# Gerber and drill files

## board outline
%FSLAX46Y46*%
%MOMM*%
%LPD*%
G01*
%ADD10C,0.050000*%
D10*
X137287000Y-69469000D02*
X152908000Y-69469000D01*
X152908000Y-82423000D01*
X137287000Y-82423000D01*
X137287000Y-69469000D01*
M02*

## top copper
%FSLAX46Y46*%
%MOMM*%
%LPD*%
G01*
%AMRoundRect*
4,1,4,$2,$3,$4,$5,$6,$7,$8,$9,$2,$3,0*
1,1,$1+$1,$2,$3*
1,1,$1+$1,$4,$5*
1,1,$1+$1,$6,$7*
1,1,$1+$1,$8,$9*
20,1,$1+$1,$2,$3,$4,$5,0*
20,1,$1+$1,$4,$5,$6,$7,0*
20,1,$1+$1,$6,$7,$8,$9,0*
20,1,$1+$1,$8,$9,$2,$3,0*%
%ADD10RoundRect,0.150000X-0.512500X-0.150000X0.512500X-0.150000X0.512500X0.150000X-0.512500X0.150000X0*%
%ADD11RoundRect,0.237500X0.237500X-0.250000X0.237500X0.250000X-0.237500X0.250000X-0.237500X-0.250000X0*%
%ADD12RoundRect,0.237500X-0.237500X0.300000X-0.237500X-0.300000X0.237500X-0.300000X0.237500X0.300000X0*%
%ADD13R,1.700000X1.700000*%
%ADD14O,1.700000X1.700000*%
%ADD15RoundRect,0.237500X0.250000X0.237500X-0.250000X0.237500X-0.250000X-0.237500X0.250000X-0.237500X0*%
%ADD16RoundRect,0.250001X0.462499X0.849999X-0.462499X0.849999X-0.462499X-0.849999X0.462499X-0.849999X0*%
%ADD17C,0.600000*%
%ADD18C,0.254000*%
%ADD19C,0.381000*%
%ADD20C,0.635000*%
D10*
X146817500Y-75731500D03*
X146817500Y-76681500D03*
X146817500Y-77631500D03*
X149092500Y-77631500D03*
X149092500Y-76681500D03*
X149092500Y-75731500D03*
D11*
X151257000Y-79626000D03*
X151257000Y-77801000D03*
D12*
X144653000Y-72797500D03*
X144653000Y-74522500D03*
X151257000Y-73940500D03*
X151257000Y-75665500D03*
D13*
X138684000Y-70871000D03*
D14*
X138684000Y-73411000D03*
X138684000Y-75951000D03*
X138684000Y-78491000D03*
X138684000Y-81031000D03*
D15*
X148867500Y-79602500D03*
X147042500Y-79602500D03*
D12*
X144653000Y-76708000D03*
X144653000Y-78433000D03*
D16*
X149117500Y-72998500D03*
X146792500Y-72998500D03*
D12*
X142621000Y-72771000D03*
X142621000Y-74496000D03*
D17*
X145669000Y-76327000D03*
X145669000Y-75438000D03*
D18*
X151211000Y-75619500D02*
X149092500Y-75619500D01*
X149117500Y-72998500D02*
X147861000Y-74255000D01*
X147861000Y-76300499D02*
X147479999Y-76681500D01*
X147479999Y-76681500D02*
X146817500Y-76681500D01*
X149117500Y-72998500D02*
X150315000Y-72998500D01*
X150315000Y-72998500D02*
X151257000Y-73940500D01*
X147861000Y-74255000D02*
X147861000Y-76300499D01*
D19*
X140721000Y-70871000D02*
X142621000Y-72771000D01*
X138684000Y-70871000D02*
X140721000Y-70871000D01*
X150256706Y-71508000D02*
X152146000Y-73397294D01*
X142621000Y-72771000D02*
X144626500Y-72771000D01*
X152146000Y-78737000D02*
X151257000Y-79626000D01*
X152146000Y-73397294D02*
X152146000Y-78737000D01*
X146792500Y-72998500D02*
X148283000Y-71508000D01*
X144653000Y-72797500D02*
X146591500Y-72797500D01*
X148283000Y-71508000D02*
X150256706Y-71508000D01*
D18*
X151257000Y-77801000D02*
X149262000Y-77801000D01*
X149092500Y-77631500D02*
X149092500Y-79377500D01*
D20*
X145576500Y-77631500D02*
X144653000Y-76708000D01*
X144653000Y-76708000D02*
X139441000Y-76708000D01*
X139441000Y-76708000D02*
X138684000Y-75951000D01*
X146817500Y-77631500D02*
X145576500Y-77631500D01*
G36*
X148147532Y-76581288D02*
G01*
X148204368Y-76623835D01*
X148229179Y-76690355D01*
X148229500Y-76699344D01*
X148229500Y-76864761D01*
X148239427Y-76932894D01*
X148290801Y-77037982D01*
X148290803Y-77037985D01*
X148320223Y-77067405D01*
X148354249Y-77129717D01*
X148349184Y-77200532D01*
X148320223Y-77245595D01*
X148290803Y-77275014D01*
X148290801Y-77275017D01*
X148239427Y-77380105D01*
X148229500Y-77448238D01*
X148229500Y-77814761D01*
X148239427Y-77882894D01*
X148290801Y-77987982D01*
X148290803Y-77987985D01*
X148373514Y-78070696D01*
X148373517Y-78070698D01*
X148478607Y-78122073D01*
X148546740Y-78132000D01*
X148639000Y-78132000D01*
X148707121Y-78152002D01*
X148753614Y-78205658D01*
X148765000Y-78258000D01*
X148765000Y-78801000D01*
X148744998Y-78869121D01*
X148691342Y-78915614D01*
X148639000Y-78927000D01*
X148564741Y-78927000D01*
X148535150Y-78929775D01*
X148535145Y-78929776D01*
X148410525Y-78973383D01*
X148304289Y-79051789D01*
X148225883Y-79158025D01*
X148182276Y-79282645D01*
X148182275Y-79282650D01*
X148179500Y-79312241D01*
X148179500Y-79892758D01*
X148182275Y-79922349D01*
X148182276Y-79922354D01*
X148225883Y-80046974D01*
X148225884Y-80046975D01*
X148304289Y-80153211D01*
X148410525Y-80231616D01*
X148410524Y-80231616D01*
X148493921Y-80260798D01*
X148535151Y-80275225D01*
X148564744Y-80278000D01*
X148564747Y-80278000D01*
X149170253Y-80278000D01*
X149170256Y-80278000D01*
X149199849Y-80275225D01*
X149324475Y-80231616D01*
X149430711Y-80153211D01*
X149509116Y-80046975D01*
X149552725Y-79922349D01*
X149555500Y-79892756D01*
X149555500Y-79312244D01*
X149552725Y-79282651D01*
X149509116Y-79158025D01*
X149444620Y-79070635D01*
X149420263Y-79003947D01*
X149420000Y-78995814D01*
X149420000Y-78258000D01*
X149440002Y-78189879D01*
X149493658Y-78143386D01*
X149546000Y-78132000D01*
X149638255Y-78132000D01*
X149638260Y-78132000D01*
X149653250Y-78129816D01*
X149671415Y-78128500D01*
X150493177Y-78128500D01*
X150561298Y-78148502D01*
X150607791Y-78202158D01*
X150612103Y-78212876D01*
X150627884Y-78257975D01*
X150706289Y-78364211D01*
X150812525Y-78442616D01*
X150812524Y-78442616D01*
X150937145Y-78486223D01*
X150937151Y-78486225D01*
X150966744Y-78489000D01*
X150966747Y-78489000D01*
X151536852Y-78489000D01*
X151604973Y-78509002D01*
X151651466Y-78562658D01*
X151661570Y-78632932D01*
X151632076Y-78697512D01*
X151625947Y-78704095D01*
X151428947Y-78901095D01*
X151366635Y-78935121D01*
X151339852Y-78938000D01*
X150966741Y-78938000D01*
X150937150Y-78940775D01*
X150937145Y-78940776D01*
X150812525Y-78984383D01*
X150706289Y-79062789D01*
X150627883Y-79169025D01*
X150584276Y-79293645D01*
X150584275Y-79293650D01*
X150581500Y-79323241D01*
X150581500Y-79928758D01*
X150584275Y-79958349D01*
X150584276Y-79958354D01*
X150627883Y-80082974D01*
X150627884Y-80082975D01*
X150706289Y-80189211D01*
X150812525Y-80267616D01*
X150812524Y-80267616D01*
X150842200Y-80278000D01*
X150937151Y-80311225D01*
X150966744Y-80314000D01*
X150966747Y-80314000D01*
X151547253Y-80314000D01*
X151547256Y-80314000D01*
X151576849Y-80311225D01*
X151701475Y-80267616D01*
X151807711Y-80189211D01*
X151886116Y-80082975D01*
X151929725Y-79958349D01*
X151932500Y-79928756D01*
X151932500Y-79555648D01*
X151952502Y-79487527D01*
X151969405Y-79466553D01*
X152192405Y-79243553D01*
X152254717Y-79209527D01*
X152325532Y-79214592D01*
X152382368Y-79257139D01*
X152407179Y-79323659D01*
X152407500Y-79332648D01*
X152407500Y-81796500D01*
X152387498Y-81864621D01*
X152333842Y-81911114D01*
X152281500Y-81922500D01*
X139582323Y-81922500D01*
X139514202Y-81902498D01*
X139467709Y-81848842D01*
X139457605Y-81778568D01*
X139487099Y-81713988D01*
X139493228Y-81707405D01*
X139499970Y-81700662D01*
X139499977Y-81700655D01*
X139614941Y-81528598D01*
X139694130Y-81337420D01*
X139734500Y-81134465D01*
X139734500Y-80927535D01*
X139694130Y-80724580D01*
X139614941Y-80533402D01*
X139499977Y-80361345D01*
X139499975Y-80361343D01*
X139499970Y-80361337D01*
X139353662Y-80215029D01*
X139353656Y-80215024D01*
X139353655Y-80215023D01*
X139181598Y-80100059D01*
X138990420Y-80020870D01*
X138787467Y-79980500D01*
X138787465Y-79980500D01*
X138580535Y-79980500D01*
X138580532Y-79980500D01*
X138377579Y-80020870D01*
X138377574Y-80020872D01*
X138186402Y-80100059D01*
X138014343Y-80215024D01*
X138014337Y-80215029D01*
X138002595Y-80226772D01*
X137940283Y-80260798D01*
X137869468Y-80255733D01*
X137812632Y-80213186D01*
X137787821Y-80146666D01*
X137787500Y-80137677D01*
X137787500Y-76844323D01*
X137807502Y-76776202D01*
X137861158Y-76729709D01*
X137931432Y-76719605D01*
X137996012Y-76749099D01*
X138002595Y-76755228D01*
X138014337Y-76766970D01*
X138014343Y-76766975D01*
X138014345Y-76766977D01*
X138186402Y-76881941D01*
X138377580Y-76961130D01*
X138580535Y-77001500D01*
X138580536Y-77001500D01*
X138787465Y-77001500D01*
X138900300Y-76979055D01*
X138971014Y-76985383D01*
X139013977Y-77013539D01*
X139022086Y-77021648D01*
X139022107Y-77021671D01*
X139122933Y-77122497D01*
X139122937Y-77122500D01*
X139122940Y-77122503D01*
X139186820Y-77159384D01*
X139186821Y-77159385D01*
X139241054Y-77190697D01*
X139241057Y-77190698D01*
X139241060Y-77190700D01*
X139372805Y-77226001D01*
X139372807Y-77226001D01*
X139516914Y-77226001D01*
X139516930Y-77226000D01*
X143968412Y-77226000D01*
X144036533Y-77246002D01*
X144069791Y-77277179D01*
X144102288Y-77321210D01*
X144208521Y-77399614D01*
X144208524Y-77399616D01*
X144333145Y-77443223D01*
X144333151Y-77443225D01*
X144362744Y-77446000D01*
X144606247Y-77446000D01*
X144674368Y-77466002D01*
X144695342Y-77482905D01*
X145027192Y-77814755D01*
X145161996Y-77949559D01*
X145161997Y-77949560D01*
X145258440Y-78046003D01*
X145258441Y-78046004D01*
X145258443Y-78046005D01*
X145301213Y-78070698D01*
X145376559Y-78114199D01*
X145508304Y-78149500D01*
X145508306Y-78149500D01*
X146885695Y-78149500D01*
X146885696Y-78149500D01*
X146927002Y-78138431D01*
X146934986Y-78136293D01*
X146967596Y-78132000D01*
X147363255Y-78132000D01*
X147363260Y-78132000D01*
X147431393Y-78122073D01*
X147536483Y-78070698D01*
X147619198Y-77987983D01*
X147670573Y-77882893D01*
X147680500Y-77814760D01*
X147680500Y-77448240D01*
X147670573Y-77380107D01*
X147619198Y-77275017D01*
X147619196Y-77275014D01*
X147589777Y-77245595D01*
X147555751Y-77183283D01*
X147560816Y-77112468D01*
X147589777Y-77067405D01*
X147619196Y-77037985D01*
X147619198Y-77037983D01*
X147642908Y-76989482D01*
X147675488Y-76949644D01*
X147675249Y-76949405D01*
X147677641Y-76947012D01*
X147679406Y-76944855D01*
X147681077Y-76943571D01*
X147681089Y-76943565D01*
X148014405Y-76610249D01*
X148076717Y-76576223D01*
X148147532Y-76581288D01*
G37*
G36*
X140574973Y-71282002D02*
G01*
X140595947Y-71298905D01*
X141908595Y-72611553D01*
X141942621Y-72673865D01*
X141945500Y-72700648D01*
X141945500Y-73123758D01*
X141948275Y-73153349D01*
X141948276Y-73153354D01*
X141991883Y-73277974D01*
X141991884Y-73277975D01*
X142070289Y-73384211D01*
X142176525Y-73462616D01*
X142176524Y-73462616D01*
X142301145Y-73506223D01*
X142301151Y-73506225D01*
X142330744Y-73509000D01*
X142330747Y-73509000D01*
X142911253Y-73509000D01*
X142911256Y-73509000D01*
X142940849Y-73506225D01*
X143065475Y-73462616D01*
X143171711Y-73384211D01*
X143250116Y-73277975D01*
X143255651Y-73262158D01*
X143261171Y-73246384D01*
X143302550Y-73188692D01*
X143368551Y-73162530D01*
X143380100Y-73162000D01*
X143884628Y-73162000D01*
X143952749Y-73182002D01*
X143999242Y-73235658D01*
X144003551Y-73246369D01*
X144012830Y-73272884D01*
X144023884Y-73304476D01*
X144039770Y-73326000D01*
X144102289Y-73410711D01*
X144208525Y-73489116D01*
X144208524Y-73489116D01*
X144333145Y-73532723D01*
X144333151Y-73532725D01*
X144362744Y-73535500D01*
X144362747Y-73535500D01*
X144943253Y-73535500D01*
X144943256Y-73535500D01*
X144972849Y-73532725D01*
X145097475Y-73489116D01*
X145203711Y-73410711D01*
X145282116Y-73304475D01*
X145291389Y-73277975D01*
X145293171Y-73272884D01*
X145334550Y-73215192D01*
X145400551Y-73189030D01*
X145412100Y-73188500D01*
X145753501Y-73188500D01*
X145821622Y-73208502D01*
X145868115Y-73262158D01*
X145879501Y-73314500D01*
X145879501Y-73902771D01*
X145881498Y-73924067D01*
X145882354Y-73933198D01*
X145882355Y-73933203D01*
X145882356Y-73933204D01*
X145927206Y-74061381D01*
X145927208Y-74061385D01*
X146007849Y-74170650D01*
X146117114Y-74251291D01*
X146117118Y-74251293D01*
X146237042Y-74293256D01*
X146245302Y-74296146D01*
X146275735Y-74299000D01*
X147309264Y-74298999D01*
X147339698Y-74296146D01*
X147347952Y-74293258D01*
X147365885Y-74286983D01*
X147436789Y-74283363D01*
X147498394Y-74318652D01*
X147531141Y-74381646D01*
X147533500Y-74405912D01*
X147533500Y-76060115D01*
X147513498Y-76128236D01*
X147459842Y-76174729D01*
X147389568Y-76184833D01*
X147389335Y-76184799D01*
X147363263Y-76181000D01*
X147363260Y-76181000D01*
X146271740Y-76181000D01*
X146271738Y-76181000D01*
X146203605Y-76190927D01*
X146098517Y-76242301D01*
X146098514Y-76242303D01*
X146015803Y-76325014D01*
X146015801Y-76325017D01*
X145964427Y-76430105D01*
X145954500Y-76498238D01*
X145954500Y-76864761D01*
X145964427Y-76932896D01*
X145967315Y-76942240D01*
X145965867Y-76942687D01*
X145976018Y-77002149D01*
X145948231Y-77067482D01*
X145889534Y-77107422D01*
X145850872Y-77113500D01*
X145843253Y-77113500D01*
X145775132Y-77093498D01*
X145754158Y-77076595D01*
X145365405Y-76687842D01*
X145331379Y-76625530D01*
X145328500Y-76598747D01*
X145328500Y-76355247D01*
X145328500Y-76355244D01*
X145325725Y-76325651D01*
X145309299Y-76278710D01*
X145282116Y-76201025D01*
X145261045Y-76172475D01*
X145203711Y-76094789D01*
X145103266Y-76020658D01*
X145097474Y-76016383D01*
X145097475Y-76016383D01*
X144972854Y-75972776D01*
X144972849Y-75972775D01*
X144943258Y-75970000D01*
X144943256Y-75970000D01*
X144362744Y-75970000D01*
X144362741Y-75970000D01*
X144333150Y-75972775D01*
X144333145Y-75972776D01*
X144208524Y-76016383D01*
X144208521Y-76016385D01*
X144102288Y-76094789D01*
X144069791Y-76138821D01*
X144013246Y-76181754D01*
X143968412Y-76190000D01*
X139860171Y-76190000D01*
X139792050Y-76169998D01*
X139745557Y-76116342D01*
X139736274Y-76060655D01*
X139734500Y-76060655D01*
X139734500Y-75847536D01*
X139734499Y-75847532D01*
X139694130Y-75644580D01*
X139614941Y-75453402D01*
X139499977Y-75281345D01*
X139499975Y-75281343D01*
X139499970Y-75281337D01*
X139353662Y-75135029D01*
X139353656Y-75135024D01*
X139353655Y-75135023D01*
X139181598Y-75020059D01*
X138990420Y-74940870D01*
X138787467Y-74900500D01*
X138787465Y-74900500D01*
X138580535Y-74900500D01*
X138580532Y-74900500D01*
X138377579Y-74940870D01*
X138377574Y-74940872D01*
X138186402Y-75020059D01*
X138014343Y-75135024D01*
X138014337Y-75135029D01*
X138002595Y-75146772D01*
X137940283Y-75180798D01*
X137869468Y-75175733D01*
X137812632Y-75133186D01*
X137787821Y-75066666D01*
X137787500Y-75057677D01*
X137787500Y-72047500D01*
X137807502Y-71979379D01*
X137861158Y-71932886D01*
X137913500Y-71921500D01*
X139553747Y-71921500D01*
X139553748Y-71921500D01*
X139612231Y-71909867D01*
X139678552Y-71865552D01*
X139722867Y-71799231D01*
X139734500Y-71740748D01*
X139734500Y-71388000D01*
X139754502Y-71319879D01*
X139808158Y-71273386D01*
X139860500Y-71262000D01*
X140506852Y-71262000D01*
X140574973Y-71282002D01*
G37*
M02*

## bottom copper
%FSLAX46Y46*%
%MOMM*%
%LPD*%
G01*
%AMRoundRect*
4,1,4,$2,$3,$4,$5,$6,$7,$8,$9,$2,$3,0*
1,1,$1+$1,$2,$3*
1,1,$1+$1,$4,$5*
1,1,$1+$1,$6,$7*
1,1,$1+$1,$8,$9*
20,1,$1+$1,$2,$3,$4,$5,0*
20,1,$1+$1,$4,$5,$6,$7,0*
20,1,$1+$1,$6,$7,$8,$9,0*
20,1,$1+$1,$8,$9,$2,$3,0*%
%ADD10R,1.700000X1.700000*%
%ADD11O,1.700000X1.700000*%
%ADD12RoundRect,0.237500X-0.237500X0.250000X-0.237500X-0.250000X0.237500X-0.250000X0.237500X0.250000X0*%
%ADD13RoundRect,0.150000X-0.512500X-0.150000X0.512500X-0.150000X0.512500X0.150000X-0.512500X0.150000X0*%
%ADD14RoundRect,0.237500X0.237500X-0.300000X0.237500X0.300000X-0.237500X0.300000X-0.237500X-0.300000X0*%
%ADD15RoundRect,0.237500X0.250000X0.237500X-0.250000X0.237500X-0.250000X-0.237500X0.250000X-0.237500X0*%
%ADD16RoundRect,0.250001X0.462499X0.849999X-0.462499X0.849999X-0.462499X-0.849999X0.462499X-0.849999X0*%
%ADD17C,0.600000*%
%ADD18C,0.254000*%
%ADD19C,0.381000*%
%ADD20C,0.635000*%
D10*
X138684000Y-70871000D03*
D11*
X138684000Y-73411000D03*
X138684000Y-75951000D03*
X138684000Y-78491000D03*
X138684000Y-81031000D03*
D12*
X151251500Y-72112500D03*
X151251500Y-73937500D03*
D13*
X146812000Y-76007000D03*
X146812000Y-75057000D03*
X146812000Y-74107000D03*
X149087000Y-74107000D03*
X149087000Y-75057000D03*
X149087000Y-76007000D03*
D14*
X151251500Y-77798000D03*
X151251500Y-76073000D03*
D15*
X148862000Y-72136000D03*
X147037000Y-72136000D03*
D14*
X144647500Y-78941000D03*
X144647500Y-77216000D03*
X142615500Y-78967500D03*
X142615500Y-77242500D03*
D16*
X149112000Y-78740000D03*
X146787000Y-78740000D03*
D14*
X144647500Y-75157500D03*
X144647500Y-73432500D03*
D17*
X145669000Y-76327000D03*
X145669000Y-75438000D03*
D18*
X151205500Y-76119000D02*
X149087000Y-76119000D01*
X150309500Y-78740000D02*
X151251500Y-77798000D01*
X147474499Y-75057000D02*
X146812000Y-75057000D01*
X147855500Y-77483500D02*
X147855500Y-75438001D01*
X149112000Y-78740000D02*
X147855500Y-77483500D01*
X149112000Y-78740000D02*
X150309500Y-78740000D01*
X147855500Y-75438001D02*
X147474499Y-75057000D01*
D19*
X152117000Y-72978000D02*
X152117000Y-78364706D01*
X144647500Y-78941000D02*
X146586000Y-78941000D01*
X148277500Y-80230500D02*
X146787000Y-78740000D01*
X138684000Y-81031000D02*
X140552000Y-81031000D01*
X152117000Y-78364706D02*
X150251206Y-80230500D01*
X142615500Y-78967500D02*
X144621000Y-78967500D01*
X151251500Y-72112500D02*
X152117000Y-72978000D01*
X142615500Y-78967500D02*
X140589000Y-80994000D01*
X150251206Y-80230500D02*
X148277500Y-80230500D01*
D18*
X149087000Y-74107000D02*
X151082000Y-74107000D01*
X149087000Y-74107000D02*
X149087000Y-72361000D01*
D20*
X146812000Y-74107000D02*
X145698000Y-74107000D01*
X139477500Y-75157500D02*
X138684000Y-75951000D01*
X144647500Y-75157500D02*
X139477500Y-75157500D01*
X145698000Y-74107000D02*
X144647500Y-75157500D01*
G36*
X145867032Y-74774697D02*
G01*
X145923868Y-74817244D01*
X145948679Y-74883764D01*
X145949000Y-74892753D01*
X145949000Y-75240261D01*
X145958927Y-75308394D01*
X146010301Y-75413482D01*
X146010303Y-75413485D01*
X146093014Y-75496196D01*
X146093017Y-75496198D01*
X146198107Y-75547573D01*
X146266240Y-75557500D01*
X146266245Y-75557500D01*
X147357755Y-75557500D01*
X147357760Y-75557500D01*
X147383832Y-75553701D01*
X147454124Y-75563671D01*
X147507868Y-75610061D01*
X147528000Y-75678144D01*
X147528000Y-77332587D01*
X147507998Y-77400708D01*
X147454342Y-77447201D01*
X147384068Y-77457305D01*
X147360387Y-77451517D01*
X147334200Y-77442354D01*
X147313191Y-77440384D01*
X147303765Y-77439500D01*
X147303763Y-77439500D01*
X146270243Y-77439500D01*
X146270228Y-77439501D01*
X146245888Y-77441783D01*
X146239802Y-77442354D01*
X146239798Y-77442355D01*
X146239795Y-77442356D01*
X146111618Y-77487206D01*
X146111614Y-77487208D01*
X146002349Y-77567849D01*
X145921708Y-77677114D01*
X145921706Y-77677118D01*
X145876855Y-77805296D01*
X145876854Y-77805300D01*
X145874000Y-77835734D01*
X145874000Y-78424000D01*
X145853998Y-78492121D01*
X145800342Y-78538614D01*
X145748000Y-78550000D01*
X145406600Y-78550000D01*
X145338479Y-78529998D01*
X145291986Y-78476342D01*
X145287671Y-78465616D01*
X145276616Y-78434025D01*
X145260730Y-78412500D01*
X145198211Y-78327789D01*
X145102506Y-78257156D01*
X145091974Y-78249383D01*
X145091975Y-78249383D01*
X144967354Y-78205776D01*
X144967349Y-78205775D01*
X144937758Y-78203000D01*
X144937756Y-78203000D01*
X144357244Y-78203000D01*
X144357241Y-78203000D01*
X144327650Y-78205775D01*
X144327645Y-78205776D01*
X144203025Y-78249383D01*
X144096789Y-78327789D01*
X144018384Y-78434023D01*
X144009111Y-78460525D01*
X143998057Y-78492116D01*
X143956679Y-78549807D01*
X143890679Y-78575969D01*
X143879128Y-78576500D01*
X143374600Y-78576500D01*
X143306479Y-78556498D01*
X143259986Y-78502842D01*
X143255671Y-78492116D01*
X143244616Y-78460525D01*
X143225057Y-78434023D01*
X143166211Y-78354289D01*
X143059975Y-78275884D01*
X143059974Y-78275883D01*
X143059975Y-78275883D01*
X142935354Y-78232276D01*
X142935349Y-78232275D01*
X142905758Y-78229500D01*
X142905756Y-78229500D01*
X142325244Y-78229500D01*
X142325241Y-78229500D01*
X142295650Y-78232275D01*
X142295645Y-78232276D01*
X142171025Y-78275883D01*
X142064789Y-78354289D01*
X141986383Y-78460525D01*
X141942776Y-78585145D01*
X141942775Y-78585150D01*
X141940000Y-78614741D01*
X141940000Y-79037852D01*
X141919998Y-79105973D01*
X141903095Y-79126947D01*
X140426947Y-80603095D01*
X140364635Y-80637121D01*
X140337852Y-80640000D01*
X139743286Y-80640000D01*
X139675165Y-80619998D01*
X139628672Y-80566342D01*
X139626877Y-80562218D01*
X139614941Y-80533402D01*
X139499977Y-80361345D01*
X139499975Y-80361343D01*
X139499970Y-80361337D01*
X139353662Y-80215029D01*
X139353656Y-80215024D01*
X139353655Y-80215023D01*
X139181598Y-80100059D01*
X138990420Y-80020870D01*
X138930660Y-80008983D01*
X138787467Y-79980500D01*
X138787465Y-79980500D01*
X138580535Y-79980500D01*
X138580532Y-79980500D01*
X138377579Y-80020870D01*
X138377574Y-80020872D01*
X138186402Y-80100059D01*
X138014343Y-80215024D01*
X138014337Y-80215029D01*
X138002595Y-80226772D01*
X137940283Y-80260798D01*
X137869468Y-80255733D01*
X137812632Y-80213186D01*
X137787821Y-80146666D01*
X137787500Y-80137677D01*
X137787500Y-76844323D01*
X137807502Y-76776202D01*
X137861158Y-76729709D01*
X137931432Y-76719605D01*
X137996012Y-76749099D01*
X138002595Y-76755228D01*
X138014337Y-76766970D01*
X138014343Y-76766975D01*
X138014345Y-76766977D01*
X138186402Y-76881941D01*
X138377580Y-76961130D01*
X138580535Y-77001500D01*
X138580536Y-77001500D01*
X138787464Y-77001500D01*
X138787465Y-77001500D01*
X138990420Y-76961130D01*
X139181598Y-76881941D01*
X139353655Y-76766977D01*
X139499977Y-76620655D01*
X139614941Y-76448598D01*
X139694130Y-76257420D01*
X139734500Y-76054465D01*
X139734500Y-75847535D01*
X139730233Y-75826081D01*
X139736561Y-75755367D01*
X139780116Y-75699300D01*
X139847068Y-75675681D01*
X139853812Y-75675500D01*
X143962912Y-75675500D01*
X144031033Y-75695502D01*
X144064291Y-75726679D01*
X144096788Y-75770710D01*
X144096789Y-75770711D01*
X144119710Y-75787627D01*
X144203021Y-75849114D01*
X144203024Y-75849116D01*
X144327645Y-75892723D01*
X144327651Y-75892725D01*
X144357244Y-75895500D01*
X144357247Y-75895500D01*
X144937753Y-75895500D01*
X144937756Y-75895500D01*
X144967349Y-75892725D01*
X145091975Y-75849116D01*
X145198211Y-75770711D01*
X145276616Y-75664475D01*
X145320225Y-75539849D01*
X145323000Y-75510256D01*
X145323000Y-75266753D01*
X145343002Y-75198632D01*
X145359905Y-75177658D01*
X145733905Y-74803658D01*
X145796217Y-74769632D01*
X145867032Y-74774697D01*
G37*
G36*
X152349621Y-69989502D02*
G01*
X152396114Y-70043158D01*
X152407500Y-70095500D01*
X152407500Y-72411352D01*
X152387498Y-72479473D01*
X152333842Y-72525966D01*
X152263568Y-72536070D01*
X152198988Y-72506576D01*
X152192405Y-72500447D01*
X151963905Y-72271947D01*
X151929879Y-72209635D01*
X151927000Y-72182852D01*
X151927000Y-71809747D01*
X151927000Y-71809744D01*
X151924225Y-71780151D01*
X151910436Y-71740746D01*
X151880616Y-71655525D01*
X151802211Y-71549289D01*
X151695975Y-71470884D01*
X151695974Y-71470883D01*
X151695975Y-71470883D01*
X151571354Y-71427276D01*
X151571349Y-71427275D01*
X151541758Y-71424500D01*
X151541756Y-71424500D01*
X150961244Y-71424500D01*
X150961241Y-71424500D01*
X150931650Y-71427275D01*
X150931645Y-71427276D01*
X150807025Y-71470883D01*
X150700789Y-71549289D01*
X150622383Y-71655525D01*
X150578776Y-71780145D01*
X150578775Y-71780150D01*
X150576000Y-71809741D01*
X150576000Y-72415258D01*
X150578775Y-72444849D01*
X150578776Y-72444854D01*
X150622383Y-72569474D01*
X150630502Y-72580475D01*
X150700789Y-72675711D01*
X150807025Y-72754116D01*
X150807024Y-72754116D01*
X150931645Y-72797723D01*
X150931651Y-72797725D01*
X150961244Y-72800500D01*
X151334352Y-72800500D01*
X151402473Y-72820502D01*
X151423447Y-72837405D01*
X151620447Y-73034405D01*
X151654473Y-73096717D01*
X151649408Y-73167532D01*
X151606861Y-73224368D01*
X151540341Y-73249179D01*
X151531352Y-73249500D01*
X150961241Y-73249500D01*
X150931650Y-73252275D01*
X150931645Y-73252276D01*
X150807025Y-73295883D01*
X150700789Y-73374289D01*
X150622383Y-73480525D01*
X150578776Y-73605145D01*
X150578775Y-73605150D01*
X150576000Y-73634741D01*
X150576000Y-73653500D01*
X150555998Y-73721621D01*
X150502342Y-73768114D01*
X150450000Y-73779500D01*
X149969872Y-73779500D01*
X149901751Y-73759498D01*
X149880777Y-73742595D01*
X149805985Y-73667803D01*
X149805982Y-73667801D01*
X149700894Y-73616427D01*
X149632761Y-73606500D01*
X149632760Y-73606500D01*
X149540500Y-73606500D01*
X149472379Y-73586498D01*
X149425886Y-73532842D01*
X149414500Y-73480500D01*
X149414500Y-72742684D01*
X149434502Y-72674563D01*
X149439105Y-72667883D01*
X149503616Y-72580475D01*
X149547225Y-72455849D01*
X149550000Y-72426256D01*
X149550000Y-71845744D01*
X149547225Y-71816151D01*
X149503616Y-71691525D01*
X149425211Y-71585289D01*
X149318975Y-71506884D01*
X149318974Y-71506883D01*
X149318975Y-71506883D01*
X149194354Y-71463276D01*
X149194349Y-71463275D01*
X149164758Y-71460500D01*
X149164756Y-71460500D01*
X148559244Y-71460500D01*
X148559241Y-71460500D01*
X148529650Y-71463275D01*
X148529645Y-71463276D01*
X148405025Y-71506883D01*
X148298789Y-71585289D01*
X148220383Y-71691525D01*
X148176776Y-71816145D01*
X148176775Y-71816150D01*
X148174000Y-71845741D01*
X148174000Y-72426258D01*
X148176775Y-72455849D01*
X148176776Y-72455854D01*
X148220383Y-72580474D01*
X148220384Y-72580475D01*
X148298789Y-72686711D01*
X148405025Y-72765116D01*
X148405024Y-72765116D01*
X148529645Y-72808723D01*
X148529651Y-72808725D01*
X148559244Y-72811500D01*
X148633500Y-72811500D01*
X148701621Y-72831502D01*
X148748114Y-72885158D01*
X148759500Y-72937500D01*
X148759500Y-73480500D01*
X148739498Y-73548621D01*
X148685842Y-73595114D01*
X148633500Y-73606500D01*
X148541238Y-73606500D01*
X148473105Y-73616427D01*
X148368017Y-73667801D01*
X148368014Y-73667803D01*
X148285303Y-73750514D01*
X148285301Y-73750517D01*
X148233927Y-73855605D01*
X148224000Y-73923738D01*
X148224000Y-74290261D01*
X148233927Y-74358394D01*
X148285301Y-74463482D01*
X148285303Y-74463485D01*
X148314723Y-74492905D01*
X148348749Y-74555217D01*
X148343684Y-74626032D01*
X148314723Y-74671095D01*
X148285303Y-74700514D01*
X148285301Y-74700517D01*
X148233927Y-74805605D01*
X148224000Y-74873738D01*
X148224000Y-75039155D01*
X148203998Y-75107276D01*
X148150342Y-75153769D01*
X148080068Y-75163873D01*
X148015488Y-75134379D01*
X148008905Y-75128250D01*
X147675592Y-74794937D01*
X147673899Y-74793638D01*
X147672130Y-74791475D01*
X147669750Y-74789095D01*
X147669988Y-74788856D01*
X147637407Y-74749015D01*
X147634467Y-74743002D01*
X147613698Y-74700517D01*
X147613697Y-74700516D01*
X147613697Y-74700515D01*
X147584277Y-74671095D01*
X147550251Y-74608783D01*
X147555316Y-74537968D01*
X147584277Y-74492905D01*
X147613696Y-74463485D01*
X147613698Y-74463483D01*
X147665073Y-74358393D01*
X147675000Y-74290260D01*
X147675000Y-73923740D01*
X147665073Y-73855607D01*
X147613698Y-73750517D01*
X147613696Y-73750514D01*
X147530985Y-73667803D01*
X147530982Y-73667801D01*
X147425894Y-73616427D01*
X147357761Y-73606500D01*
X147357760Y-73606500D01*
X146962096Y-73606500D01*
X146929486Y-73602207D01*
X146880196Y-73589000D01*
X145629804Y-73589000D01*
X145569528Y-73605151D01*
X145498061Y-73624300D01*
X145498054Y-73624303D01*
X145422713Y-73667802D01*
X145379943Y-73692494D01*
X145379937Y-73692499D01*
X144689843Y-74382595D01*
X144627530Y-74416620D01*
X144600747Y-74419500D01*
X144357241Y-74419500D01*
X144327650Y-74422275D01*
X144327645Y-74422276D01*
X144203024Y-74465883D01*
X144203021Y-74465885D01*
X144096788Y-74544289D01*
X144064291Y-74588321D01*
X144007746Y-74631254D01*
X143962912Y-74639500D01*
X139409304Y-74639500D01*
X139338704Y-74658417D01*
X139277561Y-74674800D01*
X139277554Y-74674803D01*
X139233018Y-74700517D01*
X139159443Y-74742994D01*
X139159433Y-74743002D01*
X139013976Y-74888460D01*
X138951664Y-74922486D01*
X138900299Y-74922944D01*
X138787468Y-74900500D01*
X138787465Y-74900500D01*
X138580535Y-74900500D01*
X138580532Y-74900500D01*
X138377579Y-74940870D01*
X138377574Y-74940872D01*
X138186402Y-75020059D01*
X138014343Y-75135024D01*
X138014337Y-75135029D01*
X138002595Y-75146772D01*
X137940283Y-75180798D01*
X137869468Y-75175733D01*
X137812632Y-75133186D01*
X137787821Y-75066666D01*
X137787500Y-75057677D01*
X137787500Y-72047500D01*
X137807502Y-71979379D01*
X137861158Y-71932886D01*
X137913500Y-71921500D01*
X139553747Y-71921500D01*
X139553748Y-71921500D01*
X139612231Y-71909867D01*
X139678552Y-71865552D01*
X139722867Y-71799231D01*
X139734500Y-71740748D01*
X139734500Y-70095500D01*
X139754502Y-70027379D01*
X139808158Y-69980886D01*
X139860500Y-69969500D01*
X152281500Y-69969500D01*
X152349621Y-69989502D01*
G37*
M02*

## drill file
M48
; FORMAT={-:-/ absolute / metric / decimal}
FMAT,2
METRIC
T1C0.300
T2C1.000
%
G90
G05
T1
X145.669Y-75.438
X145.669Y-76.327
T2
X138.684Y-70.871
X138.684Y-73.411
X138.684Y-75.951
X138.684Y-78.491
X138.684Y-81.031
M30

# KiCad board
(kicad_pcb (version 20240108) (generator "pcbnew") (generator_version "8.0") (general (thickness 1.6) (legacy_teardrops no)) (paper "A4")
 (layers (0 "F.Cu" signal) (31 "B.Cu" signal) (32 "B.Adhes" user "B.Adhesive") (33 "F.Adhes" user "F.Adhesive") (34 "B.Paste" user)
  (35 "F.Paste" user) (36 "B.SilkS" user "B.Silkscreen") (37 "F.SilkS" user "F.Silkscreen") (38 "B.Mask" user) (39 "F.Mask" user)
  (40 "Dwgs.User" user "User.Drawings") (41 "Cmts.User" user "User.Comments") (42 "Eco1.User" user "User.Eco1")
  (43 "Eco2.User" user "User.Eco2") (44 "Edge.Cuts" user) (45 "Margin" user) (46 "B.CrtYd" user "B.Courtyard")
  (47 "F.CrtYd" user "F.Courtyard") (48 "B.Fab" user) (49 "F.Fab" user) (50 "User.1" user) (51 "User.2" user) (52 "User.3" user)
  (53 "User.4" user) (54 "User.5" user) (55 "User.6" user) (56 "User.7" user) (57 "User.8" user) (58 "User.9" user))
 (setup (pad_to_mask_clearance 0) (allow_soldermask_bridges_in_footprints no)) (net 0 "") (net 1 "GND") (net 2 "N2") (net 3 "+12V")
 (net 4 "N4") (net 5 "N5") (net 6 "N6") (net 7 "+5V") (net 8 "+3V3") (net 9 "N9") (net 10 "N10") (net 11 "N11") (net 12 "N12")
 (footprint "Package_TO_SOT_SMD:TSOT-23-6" (layer "F.Cu") (at 147.955 76.6815)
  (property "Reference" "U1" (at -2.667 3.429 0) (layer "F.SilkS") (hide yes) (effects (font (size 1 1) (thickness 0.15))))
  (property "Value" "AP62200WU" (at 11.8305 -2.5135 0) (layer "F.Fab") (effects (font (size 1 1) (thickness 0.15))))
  (pad "1" smd roundrect (at -1.1375 -0.95) (size 1.325 0.6) (layers "F.Cu" "F.Paste" "F.Mask") (roundrect_rratio 0.25) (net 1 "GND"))
  (pad "2" smd roundrect (at -1.1375 0) (size 1.325 0.6) (layers "F.Cu" "F.Paste" "F.Mask") (roundrect_rratio 0.25) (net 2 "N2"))
  (pad "3" smd roundrect (at -1.1375 0.95) (size 1.325 0.6) (layers "F.Cu" "F.Paste" "F.Mask") (roundrect_rratio 0.25) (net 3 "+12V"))
  (pad "4" smd roundrect (at 1.1375 0.95) (size 1.325 0.6) (layers "F.Cu" "F.Paste" "F.Mask") (roundrect_rratio 0.25) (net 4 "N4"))
  (pad "5" smd roundrect (at 1.1375 0) (size 1.325 0.6) (layers "F.Cu" "F.Paste" "F.Mask") (roundrect_rratio 0.25) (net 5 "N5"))
  (pad "6" smd roundrect (at 1.1375 -0.95) (size 1.325 0.6) (layers "F.Cu" "F.Paste" "F.Mask") (roundrect_rratio 0.25) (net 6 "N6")))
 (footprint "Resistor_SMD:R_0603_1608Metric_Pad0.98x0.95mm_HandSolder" (layer "F.Cu") (at 151.257 78.7135 90)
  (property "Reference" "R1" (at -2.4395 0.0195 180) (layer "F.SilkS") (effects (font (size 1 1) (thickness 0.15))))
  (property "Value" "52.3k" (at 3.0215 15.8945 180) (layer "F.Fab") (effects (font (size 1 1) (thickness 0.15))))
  (pad "1" smd roundrect (at -0.9125 0 90) (size 0.975 0.95) (layers "F.Cu" "F.Paste" "F.Mask") (roundrect_rratio 0.25) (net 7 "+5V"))
  (pad "2" smd roundrect (at 0.9125 0 90) (size 0.975 0.95) (layers "F.Cu" "F.Paste" "F.Mask") (roundrect_rratio 0.25) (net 4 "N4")))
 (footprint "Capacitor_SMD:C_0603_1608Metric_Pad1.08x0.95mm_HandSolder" (layer "F.Cu") (at 144.653 73.66 -90)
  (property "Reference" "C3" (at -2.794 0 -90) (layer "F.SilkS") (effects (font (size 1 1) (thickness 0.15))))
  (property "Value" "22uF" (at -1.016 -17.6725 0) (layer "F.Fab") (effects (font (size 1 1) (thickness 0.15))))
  (pad "1" smd roundrect (at -0.8625 0 270) (size 1.075 0.95) (layers "F.Cu" "F.Paste" "F.Mask") (roundrect_rratio 0.25) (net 7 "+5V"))
  (pad "2" smd roundrect (at 0.8625 0 270) (size 1.075 0.95) (layers "F.Cu" "F.Paste" "F.Mask") (roundrect_rratio 0.25) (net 1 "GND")))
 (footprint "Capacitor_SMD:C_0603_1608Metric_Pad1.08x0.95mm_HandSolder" (layer "F.Cu") (at 151.257 74.803 -90)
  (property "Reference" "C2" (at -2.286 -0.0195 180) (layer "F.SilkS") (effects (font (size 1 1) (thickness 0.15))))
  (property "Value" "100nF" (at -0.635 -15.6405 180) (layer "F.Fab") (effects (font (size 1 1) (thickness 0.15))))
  (pad "1" smd roundrect (at -0.8625 0 270) (size 1.075 0.95) (layers "F.Cu" "F.Paste" "F.Mask") (roundrect_rratio 0.25) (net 2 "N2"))
  (pad "2" smd roundrect (at 0.8625 0 270) (size 1.075 0.95) (layers "F.Cu" "F.Paste" "F.Mask") (roundrect_rratio 0.25) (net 6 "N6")))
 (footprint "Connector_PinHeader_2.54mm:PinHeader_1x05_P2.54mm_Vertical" (layer "F.Cu") (at 138.684 70.871)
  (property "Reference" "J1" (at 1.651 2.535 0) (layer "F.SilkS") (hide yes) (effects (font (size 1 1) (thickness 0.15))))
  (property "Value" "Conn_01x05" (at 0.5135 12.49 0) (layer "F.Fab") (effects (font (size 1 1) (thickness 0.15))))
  (pad "1" thru_hole rect (at 0 0) (size 1.7 1.7) (drill 1) (layers "*.Cu" "*.Mask") (remove_unused_layers no) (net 7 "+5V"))
  (pad "2" thru_hole oval (at 0 2.54) (size 1.7 1.7) (drill 1) (layers "*.Cu" "*.Mask") (remove_unused_layers no) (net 1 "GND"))
  (pad "3" thru_hole oval (at 0 5.08) (size 1.7 1.7) (drill 1) (layers "*.Cu" "*.Mask") (remove_unused_layers no) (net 3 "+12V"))
  (pad "4" thru_hole oval (at 0 7.62) (size 1.7 1.7) (drill 1) (layers "*.Cu" "*.Mask") (remove_unused_layers no) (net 1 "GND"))
  (pad "5" thru_hole oval (at 0 10.16) (size 1.7 1.7) (drill 1) (layers "*.Cu" "*.Mask") (remove_unused_layers no) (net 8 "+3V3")))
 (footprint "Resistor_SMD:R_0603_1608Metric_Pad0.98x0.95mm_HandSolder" (layer "F.Cu") (at 147.955 79.6025 180)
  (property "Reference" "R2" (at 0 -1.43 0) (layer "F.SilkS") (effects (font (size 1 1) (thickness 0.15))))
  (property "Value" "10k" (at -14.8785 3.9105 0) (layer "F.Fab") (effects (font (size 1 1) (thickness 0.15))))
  (pad "1" smd roundrect (at -0.9125 0 180) (size 0.975 0.95) (layers "F.Cu" "F.Paste" "F.Mask") (roundrect_rratio 0.25) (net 4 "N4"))
  (pad "2" smd roundrect (at 0.9125 0 180) (size 0.975 0.95) (layers "F.Cu" "F.Paste" "F.Mask") (roundrect_rratio 0.25) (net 1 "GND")))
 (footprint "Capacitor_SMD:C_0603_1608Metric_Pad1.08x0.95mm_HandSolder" (layer "F.Cu") (at 144.653 77.5705 -90)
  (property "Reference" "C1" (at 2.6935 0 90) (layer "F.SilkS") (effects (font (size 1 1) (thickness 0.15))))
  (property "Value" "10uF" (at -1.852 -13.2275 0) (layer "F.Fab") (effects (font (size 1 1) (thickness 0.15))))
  (pad "1" smd roundrect (at -0.8625 0 270) (size 1.075 0.95) (layers "F.Cu" "F.Paste" "F.Mask") (roundrect_rratio 0.25) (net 3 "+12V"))
  (pad "2" smd roundrect (at 0.8625 0 270) (size 1.075 0.95) (layers "F.Cu" "F.Paste" "F.Mask") (roundrect_rratio 0.25) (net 1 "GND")))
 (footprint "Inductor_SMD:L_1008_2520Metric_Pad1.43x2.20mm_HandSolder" (layer "F.Cu") (at 147.955 72.9985 180)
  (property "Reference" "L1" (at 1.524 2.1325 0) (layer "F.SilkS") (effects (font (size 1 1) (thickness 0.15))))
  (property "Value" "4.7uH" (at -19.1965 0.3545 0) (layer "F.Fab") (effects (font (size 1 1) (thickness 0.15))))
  (pad "1" smd roundrect (at -1.1625 0 180) (size 1.425 2.2) (layers "F.Cu" "F.Paste" "F.Mask") (roundrect_rratio 0.175439) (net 2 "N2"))
  (pad "2" smd roundrect (at 1.1625 0 180) (size 1.425 2.2) (layers "F.Cu" "F.Paste" "F.Mask") (roundrect_rratio 0.175439) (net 7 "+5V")))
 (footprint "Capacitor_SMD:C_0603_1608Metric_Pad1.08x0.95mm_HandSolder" (layer "F.Cu") (at 142.621 73.6335 -90)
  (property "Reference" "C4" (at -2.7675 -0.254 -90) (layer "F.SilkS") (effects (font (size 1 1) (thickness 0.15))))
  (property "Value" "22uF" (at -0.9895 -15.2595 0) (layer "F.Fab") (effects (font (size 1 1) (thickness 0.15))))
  (pad "1" smd roundrect (at -0.8625 0 270) (size 1.075 0.95) (layers "F.Cu" "F.Paste" "F.Mask") (roundrect_rratio 0.25) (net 7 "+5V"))
  (pad "2" smd roundrect (at 0.8625 0 270) (size 1.075 0.95) (layers "F.Cu" "F.Paste" "F.Mask") (roundrect_rratio 0.25) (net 1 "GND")))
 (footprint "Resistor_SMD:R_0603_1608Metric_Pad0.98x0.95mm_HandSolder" (layer "B.Cu") (at 151.2515 73.025 -90)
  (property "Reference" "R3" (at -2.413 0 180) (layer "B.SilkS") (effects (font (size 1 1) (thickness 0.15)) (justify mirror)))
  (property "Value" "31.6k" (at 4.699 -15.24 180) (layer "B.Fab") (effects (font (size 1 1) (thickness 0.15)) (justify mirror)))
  (pad "1" smd roundrect (at -0.9125 0 270) (size 0.975 0.95) (layers "B.Cu" "B.Paste" "B.Mask") (roundrect_rratio 0.25) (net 8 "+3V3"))
  (pad "2" smd roundrect (at 0.9125 0 270) (size 0.975 0.95) (layers "B.Cu" "B.Paste" "B.Mask") (roundrect_rratio 0.25) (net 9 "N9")))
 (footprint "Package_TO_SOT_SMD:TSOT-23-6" (layer "B.Cu") (at 147.9495 75.057)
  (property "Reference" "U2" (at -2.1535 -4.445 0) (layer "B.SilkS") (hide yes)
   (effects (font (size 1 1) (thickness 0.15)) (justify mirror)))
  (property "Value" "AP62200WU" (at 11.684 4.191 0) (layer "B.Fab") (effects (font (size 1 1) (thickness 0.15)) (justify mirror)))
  (pad "1" smd roundrect (at -1.1375 0.95) (size 1.325 0.6) (layers "B.Cu" "B.Paste" "B.Mask") (roundrect_rratio 0.25) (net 1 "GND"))
  (pad "2" smd roundrect (at -1.1375 0) (size 1.325 0.6) (layers "B.Cu" "B.Paste" "B.Mask") (roundrect_rratio 0.25) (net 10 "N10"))
  (pad "3" smd roundrect (at -1.1375 -0.95) (size 1.325 0.6) (layers "B.Cu" "B.Paste" "B.Mask") (roundrect_rratio 0.25) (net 3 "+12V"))
  (pad "4" smd roundrect (at 1.1375 -0.95) (size 1.325 0.6) (layers "B.Cu" "B.Paste" "B.Mask") (roundrect_rratio 0.25) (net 9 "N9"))
  (pad "5" smd roundrect (at 1.1375 0) (size 1.325 0.6) (layers "B.Cu" "B.Paste" "B.Mask") (roundrect_rratio 0.25) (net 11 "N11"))
  (pad "6" smd roundrect (at 1.1375 0.95) (size 1.325 0.6) (layers "B.Cu" "B.Paste" "B.Mask") (roundrect_rratio 0.25) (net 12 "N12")))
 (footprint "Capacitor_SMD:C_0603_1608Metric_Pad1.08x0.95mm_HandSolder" (layer "B.Cu") (at 151.2515 76.9355 90)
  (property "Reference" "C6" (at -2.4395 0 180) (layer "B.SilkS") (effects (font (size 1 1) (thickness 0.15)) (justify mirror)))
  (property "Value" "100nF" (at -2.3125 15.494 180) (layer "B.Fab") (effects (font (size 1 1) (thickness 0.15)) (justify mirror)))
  (pad "1" smd roundrect (at -0.8625 0 90) (size 1.075 0.95) (layers "B.Cu" "B.Paste" "B.Mask") (roundrect_rratio 0.25) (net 10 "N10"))
  (pad "2" smd roundrect (at 0.8625 0 90) (size 1.075 0.95) (layers "B.Cu" "B.Paste" "B.Mask") (roundrect_rratio 0.25) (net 12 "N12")))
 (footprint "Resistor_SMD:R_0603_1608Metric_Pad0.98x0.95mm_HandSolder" (layer "B.Cu") (at 147.9495 72.136 180)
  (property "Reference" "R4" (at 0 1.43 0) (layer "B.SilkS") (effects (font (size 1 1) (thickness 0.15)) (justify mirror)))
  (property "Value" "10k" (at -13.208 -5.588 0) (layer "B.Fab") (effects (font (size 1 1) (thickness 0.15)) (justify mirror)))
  (pad "1" smd roundrect (at -0.9125 0 180) (size 0.975 0.95) (layers "B.Cu" "B.Paste" "B.Mask") (roundrect_rratio 0.25) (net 9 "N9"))
  (pad "2" smd roundrect (at 0.9125 0 180) (size 0.975 0.95) (layers "B.Cu" "B.Paste" "B.Mask") (roundrect_rratio 0.25) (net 1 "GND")))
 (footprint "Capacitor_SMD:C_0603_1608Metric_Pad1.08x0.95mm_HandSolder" (layer "B.Cu") (at 144.6475 78.0785 90)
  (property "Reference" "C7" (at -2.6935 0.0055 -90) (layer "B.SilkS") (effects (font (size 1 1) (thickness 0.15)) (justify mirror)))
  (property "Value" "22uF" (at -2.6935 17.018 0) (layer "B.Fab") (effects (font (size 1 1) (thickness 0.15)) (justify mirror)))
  (pad "1" smd roundrect (at -0.8625 0 90) (size 1.075 0.95) (layers "B.Cu" "B.Paste" "B.Mask") (roundrect_rratio 0.25) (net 8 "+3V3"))
  (pad "2" smd roundrect (at 0.8625 0 90) (size 1.075 0.95) (layers "B.Cu" "B.Paste" "B.Mask") (roundrect_rratio 0.25) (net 1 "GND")))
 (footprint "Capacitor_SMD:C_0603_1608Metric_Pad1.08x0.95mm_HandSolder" (layer "B.Cu") (at 142.6155 78.105 90)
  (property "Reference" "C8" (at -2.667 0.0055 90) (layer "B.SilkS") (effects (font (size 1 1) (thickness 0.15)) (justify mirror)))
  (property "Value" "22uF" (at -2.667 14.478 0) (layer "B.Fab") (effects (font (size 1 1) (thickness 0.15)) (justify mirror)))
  (pad "1" smd roundrect (at -0.8625 0 90) (size 1.075 0.95) (layers "B.Cu" "B.Paste" "B.Mask") (roundrect_rratio 0.25) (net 8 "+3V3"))
  (pad "2" smd roundrect (at 0.8625 0 90) (size 1.075 0.95) (layers "B.Cu" "B.Paste" "B.Mask") (roundrect_rratio 0.25) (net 1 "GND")))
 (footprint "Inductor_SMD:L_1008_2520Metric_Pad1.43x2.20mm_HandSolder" (layer "B.Cu") (at 147.9495 78.74 180)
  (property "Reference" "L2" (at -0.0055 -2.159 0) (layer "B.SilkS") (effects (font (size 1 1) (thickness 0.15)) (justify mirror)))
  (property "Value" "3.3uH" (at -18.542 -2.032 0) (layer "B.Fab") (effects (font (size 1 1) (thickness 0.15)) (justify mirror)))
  (pad "1" smd roundrect (at -1.1625 0 180) (size 1.425 2.2) (layers "B.Cu" "B.Paste" "B.Mask") (roundrect_rratio 0.175439) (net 10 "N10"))
  (pad "2" smd roundrect (at 1.1625 0 180) (size 1.425 2.2) (layers "B.Cu" "B.Paste" "B.Mask") (roundrect_rratio 0.175439) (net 8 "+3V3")))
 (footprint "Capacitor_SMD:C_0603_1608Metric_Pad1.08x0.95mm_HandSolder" (layer "B.Cu") (at 144.6475 74.295 90)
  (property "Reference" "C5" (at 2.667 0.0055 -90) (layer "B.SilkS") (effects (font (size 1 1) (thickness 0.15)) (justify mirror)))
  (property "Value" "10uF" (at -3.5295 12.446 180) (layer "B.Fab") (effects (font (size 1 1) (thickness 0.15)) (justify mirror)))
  (pad "1" smd roundrect (at -0.8625 0 90) (size 1.075 0.95) (layers "B.Cu" "B.Paste" "B.Mask") (roundrect_rratio 0.25) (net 3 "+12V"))
  (pad "2" smd roundrect (at 0.8625 0 90) (size 1.075 0.95) (layers "B.Cu" "B.Paste" "B.Mask") (roundrect_rratio 0.25) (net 1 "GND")))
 (gr_rect (start 137.287 69.469) (end 152.908 82.423) (stroke (width 0.05) (type default)) (fill none) (layer "Edge.Cuts"))
 (via (at 145.669 76.327) (size 0.6) (drill 0.3) (layers "F.Cu" "B.Cu") (free yes) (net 1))
 (via (at 145.669 75.438) (size 0.6) (drill 0.3) (layers "F.Cu" "B.Cu") (free yes) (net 1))
 (segment (start 151.211 75.6195) (end 149.0925 75.6195) (width 0.254) (layer "F.Cu") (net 6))
 (segment (start 149.1175 72.9985) (end 147.861 74.255) (width 0.254) (layer "F.Cu") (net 2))
 (segment (start 147.861 76.300499) (end 147.479999 76.6815) (width 0.254) (layer "F.Cu") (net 2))
 (segment (start 147.479999 76.6815) (end 146.8175 76.6815) (width 0.254) (layer "F.Cu") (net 2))
 (segment (start 149.1175 72.9985) (end 150.315 72.9985) (width 0.254) (layer "F.Cu") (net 2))
 (segment (start 150.315 72.9985) (end 151.257 73.9405) (width 0.254) (layer "F.Cu") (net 2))
 (segment (start 147.861 74.255) (end 147.861 76.300499) (width 0.254) (layer "F.Cu") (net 2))
 (segment (start 151.2055 76.119) (end 149.087 76.119) (width 0.254) (layer "B.Cu") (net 12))
 (segment (start 150.3095 78.74) (end 151.2515 77.798) (width 0.254) (layer "B.Cu") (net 10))
 (segment (start 147.474499 75.057) (end 146.812 75.057) (width 0.254) (layer "B.Cu") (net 10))
 (segment (start 147.8555 77.4835) (end 147.8555 75.438001) (width 0.254) (layer "B.Cu") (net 10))
 (segment (start 149.112 78.74) (end 147.8555 77.4835) (width 0.254) (layer "B.Cu") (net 10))
 (segment (start 149.112 78.74) (end 150.3095 78.74) (width 0.254) (layer "B.Cu") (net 10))
 (segment (start 147.8555 75.438001) (end 147.474499 75.057) (width 0.254) (layer "B.Cu") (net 10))
 (segment (start 140.721 70.871) (end 142.621 72.771) (width 0.381) (layer "F.Cu") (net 7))
 (segment (start 138.684 70.871) (end 140.721 70.871) (width 0.381) (layer "F.Cu") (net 7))
 (segment (start 150.256706 71.508) (end 152.146 73.397294) (width 0.381) (layer "F.Cu") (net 7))
 (segment (start 142.621 72.771) (end 144.6265 72.771) (width 0.381) (layer "F.Cu") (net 7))
 (segment (start 152.146 78.737) (end 151.257 79.626) (width 0.381) (layer "F.Cu") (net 7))
 (segment (start 152.146 73.397294) (end 152.146 78.737) (width 0.381) (layer "F.Cu") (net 7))
 (segment (start 146.7925 72.9985) (end 148.283 71.508) (width 0.381) (layer "F.Cu") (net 7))
 (segment (start 144.653 72.7975) (end 146.5915 72.7975) (width 0.381) (layer "F.Cu") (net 7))
 (segment (start 148.283 71.508) (end 150.256706 71.508) (width 0.381) (layer "F.Cu") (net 7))
 (segment (start 152.117 72.978) (end 152.117 78.364706) (width 0.381) (layer "B.Cu") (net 8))
 (segment (start 144.6475 78.941) (end 146.586 78.941) (width 0.381) (layer "B.Cu") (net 8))
 (segment (start 148.2775 80.2305) (end 146.787 78.74) (width 0.381) (layer "B.Cu") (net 8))
 (segment (start 138.684 81.031) (end 140.552 81.031) (width 0.381) (layer "B.Cu") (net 8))
 (segment (start 152.117 78.364706) (end 150.251206 80.2305) (width 0.381) (layer "B.Cu") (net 8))
 (segment (start 142.6155 78.9675) (end 144.621 78.9675) (width 0.381) (layer "B.Cu") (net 8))
 (segment (start 151.2515 72.1125) (end 152.117 72.978) (width 0.381) (layer "B.Cu") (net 8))
 (segment (start 142.6155 78.9675) (end 140.589 80.994) (width 0.381) (layer "B.Cu") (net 8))
 (segment (start 150.251206 80.2305) (end 148.2775 80.2305) (width 0.381) (layer "B.Cu") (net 8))
 (segment (start 151.257 77.801) (end 149.262 77.801) (width 0.254) (layer "F.Cu") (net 4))
 (segment (start 149.0925 77.6315) (end 149.0925 79.3775) (width 0.254) (layer "F.Cu") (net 4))
 (segment (start 149.087 74.107) (end 151.082 74.107) (width 0.254) (layer "B.Cu") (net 9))
 (segment (start 149.087 74.107) (end 149.087 72.361) (width 0.254) (layer "B.Cu") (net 9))
 (segment (start 145.5765 77.6315) (end 144.653 76.708) (width 0.635) (layer "F.Cu") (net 3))
 (segment (start 144.653 76.708) (end 139.441 76.708) (width 0.635) (layer "F.Cu") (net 3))
 (segment (start 139.441 76.708) (end 138.684 75.951) (width 0.635) (layer "F.Cu") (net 3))
 (segment (start 146.8175 77.6315) (end 145.5765 77.6315) (width 0.635) (layer "F.Cu") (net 3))
 (segment (start 146.812 74.107) (end 145.698 74.107) (width 0.635) (layer "B.Cu") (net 3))
 (segment (start 139.4775 75.1575) (end 138.684 75.951) (width 0.635) (layer "B.Cu") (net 3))
 (segment (start 144.6475 75.1575) (end 139.4775 75.1575) (width 0.635) (layer "B.Cu") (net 3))
 (segment (start 145.698 74.107) (end 144.6475 75.1575) (width 0.635) (layer "B.Cu") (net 3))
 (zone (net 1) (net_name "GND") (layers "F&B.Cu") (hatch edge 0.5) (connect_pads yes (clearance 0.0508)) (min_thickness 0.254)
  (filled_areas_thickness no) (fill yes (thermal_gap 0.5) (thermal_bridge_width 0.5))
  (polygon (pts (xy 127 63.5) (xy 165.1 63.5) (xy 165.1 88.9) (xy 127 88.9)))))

